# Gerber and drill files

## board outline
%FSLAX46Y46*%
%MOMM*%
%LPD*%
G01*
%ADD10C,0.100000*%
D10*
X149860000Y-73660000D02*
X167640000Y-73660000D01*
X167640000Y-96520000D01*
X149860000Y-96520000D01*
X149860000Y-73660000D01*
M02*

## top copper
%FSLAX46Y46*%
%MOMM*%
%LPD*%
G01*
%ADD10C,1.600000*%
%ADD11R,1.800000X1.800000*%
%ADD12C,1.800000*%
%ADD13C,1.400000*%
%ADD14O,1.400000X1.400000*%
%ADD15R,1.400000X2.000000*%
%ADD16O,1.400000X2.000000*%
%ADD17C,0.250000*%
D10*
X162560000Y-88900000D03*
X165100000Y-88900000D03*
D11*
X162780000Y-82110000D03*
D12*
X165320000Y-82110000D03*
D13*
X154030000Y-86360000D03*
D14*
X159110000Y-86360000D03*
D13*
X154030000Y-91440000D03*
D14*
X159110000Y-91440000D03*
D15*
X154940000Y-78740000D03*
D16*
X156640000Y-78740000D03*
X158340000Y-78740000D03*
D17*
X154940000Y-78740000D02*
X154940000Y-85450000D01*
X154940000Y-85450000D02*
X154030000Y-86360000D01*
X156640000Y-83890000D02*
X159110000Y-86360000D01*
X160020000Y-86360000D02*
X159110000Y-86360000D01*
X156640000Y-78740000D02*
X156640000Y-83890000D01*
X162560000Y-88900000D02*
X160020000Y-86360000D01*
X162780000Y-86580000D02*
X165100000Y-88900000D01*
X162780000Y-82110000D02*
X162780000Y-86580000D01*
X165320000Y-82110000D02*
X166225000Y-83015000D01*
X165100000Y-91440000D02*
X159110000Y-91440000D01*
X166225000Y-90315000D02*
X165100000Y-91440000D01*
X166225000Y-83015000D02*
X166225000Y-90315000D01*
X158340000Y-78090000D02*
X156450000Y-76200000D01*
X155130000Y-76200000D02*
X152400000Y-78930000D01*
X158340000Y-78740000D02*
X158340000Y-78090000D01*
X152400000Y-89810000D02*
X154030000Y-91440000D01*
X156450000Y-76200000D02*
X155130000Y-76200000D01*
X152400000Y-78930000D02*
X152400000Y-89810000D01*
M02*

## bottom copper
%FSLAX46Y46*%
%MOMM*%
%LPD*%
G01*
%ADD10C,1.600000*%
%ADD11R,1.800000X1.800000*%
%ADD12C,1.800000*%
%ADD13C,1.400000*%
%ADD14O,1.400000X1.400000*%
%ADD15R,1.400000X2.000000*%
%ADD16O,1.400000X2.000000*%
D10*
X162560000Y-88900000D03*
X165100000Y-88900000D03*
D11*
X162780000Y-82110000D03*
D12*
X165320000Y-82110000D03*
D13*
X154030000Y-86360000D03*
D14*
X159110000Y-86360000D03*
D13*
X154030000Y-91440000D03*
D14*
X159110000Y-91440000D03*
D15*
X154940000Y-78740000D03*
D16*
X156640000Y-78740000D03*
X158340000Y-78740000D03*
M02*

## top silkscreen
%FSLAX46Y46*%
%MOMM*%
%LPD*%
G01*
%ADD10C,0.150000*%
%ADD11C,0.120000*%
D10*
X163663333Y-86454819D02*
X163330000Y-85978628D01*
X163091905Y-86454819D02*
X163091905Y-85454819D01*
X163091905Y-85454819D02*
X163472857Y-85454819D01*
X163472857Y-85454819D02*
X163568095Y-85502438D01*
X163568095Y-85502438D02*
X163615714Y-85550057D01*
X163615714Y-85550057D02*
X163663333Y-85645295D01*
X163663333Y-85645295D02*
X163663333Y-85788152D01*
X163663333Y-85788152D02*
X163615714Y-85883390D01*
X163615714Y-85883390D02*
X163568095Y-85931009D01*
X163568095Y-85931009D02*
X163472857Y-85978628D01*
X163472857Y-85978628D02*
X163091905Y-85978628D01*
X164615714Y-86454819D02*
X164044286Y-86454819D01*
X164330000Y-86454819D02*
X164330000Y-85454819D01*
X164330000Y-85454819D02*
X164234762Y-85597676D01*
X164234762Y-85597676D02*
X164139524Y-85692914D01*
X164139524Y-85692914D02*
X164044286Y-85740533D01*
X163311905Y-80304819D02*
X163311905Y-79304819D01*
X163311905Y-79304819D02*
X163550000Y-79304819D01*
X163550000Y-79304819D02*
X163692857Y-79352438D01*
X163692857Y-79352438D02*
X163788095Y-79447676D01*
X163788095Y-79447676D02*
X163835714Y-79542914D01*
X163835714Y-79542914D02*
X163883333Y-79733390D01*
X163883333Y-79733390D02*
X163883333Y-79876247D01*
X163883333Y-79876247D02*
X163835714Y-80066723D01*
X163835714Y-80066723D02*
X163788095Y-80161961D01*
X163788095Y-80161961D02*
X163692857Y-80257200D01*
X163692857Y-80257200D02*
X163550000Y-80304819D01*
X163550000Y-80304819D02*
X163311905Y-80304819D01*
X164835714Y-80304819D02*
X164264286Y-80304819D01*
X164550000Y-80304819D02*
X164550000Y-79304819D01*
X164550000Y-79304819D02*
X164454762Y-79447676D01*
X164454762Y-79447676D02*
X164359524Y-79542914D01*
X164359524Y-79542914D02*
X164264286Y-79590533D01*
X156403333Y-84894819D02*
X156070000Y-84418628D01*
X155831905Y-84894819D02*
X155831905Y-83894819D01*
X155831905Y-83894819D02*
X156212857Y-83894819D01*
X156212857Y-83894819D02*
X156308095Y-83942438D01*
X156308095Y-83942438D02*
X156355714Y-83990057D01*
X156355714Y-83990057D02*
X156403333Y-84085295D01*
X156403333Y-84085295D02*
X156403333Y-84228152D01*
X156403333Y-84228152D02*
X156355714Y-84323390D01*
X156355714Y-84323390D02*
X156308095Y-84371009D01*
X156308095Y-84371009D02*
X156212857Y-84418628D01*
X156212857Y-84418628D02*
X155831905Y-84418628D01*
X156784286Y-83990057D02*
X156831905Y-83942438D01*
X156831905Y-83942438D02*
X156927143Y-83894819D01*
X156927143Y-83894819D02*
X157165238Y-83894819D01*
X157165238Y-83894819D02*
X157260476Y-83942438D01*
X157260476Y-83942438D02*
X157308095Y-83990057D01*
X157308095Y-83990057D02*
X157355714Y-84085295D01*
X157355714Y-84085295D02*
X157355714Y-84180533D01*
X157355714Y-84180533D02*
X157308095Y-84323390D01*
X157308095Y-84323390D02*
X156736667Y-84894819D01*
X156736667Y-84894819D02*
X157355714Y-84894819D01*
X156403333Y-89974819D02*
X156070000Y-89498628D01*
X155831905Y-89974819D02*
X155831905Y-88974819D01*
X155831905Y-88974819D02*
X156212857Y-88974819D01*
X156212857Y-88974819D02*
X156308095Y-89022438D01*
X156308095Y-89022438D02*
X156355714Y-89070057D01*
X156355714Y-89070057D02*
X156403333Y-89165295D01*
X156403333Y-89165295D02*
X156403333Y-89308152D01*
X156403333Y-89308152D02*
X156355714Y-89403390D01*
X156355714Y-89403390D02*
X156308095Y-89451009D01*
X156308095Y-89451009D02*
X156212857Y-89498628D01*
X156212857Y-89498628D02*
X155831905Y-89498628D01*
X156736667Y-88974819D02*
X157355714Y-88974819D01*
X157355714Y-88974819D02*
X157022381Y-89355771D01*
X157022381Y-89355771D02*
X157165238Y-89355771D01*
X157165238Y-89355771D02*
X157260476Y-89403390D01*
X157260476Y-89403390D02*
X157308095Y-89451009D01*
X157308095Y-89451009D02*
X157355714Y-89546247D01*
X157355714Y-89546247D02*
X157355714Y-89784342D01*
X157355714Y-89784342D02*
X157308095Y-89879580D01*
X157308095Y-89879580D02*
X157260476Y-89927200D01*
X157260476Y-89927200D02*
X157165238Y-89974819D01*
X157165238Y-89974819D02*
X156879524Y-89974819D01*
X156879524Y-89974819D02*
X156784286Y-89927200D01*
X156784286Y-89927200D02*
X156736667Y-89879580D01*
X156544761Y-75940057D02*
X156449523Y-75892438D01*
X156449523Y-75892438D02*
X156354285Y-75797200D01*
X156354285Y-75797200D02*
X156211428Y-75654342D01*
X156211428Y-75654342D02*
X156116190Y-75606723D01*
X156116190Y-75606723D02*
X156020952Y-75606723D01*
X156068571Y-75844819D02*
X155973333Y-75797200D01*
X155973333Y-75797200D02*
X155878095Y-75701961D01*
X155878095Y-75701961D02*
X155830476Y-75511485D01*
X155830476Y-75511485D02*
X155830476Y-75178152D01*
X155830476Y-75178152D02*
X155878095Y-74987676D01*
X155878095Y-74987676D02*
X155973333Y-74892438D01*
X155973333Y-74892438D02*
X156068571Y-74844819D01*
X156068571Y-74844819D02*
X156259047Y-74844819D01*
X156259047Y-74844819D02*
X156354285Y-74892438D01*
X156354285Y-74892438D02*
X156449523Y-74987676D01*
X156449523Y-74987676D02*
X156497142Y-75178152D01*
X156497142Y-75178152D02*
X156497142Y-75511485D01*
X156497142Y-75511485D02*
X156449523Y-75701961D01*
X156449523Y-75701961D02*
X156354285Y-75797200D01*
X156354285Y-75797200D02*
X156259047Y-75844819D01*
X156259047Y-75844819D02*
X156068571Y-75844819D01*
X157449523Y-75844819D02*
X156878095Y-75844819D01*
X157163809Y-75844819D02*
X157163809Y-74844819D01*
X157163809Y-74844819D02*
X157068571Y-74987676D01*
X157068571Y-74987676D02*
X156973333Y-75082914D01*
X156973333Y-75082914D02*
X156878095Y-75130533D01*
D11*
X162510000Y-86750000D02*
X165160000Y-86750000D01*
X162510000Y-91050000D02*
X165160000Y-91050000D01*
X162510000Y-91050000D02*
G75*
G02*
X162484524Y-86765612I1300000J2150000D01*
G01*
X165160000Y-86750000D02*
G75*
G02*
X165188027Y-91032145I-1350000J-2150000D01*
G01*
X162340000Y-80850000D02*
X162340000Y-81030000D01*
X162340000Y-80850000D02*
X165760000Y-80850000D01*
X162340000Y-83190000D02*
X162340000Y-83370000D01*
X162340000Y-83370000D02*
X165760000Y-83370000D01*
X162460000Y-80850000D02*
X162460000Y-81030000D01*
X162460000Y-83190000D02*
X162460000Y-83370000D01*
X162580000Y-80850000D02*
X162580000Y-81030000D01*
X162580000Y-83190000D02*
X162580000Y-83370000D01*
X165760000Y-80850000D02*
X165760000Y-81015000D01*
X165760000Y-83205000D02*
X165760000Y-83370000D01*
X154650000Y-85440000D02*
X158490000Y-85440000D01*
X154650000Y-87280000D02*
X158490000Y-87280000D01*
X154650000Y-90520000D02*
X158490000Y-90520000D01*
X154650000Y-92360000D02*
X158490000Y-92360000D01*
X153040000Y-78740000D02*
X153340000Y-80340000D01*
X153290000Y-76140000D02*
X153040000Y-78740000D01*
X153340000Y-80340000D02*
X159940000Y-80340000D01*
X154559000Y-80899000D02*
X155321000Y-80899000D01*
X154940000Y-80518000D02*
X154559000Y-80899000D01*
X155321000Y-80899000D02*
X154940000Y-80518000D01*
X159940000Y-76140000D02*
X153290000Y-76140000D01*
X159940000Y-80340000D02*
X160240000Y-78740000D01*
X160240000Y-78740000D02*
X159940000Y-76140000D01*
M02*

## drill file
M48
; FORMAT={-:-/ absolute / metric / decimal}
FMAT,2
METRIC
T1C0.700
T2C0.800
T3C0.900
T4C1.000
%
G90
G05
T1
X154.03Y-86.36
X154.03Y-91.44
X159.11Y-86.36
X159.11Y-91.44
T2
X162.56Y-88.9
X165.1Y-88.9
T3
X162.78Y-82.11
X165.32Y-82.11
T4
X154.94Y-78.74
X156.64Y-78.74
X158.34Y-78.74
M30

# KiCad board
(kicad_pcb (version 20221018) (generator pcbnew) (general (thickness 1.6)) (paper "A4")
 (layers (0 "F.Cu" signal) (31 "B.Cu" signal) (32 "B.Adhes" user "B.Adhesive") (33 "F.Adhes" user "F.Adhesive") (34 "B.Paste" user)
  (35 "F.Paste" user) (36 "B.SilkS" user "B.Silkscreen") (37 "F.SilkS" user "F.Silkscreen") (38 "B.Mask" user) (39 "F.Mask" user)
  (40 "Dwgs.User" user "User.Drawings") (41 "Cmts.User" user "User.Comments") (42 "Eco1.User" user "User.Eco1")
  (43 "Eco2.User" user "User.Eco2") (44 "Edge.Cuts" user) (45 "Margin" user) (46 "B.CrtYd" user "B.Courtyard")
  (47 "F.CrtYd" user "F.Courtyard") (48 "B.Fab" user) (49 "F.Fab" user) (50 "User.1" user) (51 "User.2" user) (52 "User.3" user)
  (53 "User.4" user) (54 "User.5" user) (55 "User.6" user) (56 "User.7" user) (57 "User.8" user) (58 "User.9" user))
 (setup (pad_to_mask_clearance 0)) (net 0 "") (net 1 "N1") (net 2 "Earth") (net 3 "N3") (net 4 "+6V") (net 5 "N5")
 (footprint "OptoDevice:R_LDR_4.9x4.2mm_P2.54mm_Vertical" (layer "F.Cu") (at 162.56 88.9)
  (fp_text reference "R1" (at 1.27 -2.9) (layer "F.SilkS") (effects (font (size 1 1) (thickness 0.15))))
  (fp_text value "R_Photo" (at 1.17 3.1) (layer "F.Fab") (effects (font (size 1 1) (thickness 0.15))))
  (fp_line (start -0.05 -2.15) (end 2.6 -2.15) (stroke (width 0.12) (type solid)) (layer "F.SilkS"))
  (fp_line (start -0.05 2.15) (end 2.6 2.15) (stroke (width 0.12) (type solid)) (layer "F.SilkS"))
  (fp_arc (start -0.05 2.15) (mid -1.262424 0.01494) (end -0.075476 -2.134388) (stroke (width 0.12) (type solid)) (layer "F.SilkS"))
  (fp_arc (start 2.6 -2.15) (mid 3.788646 -0.016616) (end 2.628027 2.132145) (stroke (width 0.12) (type solid)) (layer "F.SilkS"))
  (pad "1" thru_hole circle (at 0 0) (size 1.6 1.6) (drill 0.8) (layers "*.Cu" "*.Mask") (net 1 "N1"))
  (pad "2" thru_hole circle (at 2.54 0) (size 1.6 1.6) (drill 0.8) (layers "*.Cu" "*.Mask") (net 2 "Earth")))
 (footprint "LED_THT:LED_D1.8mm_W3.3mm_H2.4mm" (layer "F.Cu") (at 162.78 82.11)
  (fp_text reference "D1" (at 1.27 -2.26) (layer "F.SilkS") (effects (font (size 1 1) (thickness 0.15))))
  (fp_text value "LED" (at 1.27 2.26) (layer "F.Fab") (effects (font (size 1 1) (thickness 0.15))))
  (fp_line (start -0.44 -1.26) (end -0.44 -1.08) (stroke (width 0.12) (type solid)) (layer "F.SilkS"))
  (fp_line (start -0.44 -1.26) (end 2.98 -1.26) (stroke (width 0.12) (type solid)) (layer "F.SilkS"))
  (fp_line (start -0.44 1.08) (end -0.44 1.26) (stroke (width 0.12) (type solid)) (layer "F.SilkS"))
  (fp_line (start -0.44 1.26) (end 2.98 1.26) (stroke (width 0.12) (type solid)) (layer "F.SilkS"))
  (fp_line (start -0.32 -1.26) (end -0.32 -1.08) (stroke (width 0.12) (type solid)) (layer "F.SilkS"))
  (fp_line (start -0.32 1.08) (end -0.32 1.26) (stroke (width 0.12) (type solid)) (layer "F.SilkS"))
  (fp_line (start -0.2 -1.26) (end -0.2 -1.08) (stroke (width 0.12) (type solid)) (layer "F.SilkS"))
  (fp_line (start -0.2 1.08) (end -0.2 1.26) (stroke (width 0.12) (type solid)) (layer "F.SilkS"))
  (fp_line (start 2.98 -1.26) (end 2.98 -1.095) (stroke (width 0.12) (type solid)) (layer "F.SilkS"))
  (fp_line (start 2.98 1.095) (end 2.98 1.26) (stroke (width 0.12) (type solid)) (layer "F.SilkS"))
  (pad "1" thru_hole rect (at 0 0) (size 1.8 1.8) (drill 0.9) (layers "*.Cu" "*.Mask") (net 2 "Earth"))
  (pad "2" thru_hole circle (at 2.54 0) (size 1.8 1.8) (drill 0.9) (layers "*.Cu" "*.Mask") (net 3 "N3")))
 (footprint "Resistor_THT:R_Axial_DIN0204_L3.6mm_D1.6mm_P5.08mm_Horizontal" (layer "F.Cu") (at 154.03 86.36)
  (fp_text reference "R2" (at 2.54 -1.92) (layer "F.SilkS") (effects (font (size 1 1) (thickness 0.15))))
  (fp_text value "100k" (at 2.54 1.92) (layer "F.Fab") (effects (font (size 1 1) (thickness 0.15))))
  (fp_line (start 0.62 -0.92) (end 4.46 -0.92) (stroke (width 0.12) (type solid)) (layer "F.SilkS"))
  (fp_line (start 0.62 0.92) (end 4.46 0.92) (stroke (width 0.12) (type solid)) (layer "F.SilkS"))
  (pad "1" thru_hole circle (at 0 0) (size 1.4 1.4) (drill 0.7) (layers "*.Cu" "*.Mask") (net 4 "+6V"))
  (pad "2" thru_hole oval (at 5.08 0) (size 1.4 1.4) (drill 0.7) (layers "*.Cu" "*.Mask") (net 1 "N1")))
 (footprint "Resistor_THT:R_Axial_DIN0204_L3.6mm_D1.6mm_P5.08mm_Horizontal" (layer "F.Cu") (at 154.03 91.44)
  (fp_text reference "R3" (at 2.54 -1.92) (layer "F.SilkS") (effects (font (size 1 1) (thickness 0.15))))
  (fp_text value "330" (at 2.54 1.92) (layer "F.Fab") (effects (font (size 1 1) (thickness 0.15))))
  (fp_line (start 0.62 -0.92) (end 4.46 -0.92) (stroke (width 0.12) (type solid)) (layer "F.SilkS"))
  (fp_line (start 0.62 0.92) (end 4.46 0.92) (stroke (width 0.12) (type solid)) (layer "F.SilkS"))
  (pad "1" thru_hole circle (at 0 0) (size 1.4 1.4) (drill 0.7) (layers "*.Cu" "*.Mask") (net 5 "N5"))
  (pad "2" thru_hole oval (at 5.08 0) (size 1.4 1.4) (drill 0.7) (layers "*.Cu" "*.Mask") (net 3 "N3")))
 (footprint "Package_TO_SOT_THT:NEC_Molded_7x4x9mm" (layer "F.Cu") (at 154.94 78.74)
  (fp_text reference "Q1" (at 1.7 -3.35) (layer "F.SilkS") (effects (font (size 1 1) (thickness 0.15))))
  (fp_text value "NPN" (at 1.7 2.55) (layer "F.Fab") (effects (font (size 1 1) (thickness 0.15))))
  (fp_line (start -1.9 0) (end -1.6 1.6) (stroke (width 0.12) (type solid)) (layer "F.SilkS"))
  (fp_line (start -1.65 -2.6) (end -1.9 0) (stroke (width 0.12) (type solid)) (layer "F.SilkS"))
  (fp_line (start -1.6 1.6) (end 5 1.6) (stroke (width 0.12) (type solid)) (layer "F.SilkS"))
  (fp_line (start -0.381 2.159) (end 0.381 2.159) (stroke (width 0.12) (type solid)) (layer "F.SilkS"))
  (fp_line (start 0 1.778) (end -0.381 2.159) (stroke (width 0.12) (type solid)) (layer "F.SilkS"))
  (fp_line (start 0.381 2.159) (end 0 1.778) (stroke (width 0.12) (type solid)) (layer "F.SilkS"))
  (fp_line (start 5 -2.6) (end -1.65 -2.6) (stroke (width 0.12) (type solid)) (layer "F.SilkS"))
  (fp_line (start 5 1.6) (end 5.3 0) (stroke (width 0.12) (type solid)) (layer "F.SilkS"))
  (fp_line (start 5.3 0) (end 5 -2.6) (stroke (width 0.12) (type solid)) (layer "F.SilkS"))
  (pad "1" thru_hole rect (at 0 0 180) (size 1.4 2) (drill 1) (layers "*.Cu" "*.Mask") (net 4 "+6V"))
  (pad "2" thru_hole oval (at 1.7 0 180) (size 1.4 2) (drill 1) (layers "*.Cu" "*.Mask") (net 1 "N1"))
  (pad "3" thru_hole oval (at 3.4 0 180) (size 1.4 2) (drill 1) (layers "*.Cu" "*.Mask") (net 5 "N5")))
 (gr_rect (start 149.86 73.66) (end 167.64 96.52) (stroke (width 0.1) (type default)) (fill none) (layer "Edge.Cuts"))
 (segment (start 154.94 78.74) (end 154.94 85.45) (width 0.25) (layer "F.Cu") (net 4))
 (segment (start 154.94 85.45) (end 154.03 86.36) (width 0.25) (layer "F.Cu") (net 4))
 (segment (start 156.64 83.89) (end 159.11 86.36) (width 0.25) (layer "F.Cu") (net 1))
 (segment (start 160.02 86.36) (end 159.11 86.36) (width 0.25) (layer "F.Cu") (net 1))
 (segment (start 156.64 78.74) (end 156.64 83.89) (width 0.25) (layer "F.Cu") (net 1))
 (segment (start 162.56 88.9) (end 160.02 86.36) (width 0.25) (layer "F.Cu") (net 1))
 (segment (start 162.78 86.58) (end 165.1 88.9) (width 0.25) (layer "F.Cu") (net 2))
 (segment (start 162.78 82.11) (end 162.78 86.58) (width 0.25) (layer "F.Cu") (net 2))
 (segment (start 165.32 82.11) (end 166.225 83.015) (width 0.25) (layer "F.Cu") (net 3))
 (segment (start 165.1 91.44) (end 159.11 91.44) (width 0.25) (layer "F.Cu") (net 3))
 (segment (start 166.225 90.315) (end 165.1 91.44) (width 0.25) (layer "F.Cu") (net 3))
 (segment (start 166.225 83.015) (end 166.225 90.315) (width 0.25) (layer "F.Cu") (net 3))
 (segment (start 158.34 78.09) (end 156.45 76.2) (width 0.25) (layer "F.Cu") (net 5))
 (segment (start 155.13 76.2) (end 152.4 78.93) (width 0.25) (layer "F.Cu") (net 5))
 (segment (start 158.34 78.74) (end 158.34 78.09) (width 0.25) (layer "F.Cu") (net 5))
 (segment (start 152.4 89.81) (end 154.03 91.44) (width 0.25) (layer "F.Cu") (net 5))
 (segment (start 156.45 76.2) (end 155.13 76.2) (width 0.25) (layer "F.Cu") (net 5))
 (segment (start 152.4 78.93) (end 152.4 89.81) (width 0.25) (layer "F.Cu") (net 5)))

